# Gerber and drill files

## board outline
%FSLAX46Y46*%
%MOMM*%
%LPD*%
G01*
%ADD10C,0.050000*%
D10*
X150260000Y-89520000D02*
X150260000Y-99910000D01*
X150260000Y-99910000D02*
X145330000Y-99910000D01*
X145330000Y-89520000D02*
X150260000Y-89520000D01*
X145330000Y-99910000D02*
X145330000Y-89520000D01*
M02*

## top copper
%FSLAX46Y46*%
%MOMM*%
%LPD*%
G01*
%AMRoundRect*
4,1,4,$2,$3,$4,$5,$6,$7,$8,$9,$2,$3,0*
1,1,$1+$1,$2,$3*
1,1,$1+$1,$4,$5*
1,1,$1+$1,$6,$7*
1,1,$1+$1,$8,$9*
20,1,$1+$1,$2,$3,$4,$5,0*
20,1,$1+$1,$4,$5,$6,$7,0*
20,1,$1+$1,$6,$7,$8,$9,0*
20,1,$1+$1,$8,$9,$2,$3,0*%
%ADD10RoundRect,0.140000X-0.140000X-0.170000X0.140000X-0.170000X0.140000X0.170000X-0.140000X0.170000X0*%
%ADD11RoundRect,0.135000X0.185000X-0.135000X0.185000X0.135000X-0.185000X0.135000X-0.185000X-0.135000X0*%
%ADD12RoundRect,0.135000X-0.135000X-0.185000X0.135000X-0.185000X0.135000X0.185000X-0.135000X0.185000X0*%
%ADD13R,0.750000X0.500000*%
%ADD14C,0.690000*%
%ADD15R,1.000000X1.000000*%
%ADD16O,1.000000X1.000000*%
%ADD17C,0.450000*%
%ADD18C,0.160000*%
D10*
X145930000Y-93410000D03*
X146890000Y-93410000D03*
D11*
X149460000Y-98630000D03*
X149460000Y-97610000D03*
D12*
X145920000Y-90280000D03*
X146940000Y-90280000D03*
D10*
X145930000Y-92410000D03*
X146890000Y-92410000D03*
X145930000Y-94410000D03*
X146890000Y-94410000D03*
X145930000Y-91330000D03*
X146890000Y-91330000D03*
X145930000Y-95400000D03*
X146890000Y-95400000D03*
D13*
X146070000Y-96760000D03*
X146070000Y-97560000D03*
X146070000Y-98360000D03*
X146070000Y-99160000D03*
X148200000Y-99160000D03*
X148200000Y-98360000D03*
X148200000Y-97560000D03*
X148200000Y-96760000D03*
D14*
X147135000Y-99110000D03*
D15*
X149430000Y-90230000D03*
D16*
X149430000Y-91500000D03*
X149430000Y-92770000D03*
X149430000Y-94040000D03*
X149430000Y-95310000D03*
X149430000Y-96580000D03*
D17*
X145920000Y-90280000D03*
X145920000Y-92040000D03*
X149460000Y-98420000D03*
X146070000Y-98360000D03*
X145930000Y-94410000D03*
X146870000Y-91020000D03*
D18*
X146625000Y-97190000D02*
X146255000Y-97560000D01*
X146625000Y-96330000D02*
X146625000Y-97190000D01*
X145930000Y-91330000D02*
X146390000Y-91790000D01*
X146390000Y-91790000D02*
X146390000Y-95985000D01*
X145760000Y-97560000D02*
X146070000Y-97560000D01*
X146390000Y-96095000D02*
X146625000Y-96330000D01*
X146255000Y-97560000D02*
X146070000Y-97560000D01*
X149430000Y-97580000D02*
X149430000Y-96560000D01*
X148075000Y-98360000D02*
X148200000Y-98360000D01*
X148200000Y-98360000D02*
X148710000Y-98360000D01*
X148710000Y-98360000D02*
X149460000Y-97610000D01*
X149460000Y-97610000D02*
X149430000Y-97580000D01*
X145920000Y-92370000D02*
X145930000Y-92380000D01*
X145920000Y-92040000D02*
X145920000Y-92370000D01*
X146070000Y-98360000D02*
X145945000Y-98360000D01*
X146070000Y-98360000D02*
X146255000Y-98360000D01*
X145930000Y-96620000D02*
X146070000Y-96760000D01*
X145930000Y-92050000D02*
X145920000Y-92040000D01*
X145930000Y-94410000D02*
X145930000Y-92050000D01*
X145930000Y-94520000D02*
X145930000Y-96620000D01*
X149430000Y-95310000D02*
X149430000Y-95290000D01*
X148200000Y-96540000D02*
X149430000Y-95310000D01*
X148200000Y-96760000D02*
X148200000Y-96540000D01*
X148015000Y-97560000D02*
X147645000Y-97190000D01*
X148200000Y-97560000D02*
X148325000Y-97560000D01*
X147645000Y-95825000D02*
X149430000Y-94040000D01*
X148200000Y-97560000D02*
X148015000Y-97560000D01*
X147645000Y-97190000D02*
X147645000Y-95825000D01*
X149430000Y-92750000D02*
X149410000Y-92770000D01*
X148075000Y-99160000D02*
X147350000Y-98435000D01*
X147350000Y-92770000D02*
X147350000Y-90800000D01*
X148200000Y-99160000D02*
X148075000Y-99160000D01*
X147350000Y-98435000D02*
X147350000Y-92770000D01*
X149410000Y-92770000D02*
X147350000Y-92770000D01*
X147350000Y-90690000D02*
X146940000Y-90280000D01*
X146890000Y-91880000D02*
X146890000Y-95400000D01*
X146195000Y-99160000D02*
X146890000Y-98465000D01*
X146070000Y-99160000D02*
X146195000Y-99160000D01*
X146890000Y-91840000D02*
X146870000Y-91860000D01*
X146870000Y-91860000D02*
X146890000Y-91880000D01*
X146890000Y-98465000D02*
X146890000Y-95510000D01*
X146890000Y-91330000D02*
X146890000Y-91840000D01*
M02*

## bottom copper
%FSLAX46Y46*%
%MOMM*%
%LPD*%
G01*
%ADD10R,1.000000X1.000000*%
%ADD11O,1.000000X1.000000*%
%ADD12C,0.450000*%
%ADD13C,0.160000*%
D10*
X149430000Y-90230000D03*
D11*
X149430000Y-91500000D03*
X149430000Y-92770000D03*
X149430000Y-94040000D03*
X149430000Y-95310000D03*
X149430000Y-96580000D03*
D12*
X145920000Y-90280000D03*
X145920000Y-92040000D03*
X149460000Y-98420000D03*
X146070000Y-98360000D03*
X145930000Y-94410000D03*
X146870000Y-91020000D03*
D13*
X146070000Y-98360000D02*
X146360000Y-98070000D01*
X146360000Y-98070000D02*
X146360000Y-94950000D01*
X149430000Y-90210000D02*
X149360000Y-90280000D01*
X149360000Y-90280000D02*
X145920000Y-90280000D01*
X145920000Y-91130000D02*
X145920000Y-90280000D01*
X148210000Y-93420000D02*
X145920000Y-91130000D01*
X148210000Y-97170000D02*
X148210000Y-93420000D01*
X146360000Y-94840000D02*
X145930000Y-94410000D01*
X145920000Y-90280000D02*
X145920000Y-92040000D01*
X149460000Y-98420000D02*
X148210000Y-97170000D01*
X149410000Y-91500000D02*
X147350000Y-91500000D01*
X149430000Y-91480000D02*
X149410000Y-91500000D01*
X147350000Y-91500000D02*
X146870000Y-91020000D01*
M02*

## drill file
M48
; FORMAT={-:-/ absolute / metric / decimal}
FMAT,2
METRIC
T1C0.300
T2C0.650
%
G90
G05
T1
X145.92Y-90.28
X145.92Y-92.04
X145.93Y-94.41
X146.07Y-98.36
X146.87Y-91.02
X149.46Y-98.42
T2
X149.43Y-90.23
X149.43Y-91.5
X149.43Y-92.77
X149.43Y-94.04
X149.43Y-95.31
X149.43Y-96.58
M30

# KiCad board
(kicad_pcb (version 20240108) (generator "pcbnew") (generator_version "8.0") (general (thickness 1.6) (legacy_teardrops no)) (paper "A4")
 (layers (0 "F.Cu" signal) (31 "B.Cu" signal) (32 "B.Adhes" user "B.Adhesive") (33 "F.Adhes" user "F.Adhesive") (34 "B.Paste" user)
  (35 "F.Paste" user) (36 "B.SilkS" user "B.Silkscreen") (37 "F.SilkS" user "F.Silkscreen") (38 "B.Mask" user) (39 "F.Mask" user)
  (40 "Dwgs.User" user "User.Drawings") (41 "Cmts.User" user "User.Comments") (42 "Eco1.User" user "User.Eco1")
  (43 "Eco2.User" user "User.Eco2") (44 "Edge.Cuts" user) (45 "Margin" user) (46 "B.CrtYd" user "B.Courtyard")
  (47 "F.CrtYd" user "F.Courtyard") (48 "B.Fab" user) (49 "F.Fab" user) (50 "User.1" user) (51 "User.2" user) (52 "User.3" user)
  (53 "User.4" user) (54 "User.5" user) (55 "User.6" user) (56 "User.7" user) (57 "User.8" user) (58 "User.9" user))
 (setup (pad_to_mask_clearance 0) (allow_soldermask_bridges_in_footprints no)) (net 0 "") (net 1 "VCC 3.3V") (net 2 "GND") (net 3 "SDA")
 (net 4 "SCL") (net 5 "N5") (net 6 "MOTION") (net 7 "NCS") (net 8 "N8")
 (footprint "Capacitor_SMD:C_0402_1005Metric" (layer "F.Cu") (at 146.41 93.41)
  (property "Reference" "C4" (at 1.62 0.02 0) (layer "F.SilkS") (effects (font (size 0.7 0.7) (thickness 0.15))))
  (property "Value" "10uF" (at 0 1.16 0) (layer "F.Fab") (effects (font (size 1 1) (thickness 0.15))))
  (pad "1" smd roundrect (at -0.48 0) (size 0.56 0.62) (layers "F.Cu" "F.Paste" "F.Mask") (roundrect_rratio 0.25) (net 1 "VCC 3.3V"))
  (pad "2" smd roundrect (at 0.48 0) (size 0.56 0.62) (layers "F.Cu" "F.Paste" "F.Mask") (roundrect_rratio 0.25) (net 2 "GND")))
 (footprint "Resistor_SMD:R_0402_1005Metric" (layer "F.Cu") (at 149.46 98.12 90)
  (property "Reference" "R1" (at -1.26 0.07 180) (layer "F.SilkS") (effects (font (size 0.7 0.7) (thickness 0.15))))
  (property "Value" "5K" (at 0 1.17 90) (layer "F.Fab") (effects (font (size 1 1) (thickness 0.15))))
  (pad "1" smd roundrect (at -0.51 0 90) (size 0.54 0.64) (layers "F.Cu" "F.Paste" "F.Mask") (roundrect_rratio 0.25) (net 1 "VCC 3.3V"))
  (pad "2" smd roundrect (at 0.51 0 90) (size 0.54 0.64) (layers "F.Cu" "F.Paste" "F.Mask") (roundrect_rratio 0.25) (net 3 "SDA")))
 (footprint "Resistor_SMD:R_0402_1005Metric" (layer "F.Cu") (at 146.43 90.28)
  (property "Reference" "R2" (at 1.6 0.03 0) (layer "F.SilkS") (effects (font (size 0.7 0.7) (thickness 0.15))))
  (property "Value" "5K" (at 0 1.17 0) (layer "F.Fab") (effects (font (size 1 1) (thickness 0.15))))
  (pad "1" smd roundrect (at -0.51 0) (size 0.54 0.64) (layers "F.Cu" "F.Paste" "F.Mask") (roundrect_rratio 0.25) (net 1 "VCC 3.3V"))
  (pad "2" smd roundrect (at 0.51 0) (size 0.54 0.64) (layers "F.Cu" "F.Paste" "F.Mask") (roundrect_rratio 0.25) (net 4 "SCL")))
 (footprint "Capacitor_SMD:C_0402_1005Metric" (layer "F.Cu") (at 146.41 92.41)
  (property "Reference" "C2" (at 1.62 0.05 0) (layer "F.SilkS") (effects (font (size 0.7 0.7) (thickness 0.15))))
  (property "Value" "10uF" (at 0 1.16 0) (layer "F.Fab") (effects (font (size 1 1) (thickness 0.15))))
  (pad "1" smd roundrect (at -0.48 0) (size 0.56 0.62) (layers "F.Cu" "F.Paste" "F.Mask") (roundrect_rratio 0.25) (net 1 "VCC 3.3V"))
  (pad "2" smd roundrect (at 0.48 0) (size 0.56 0.62) (layers "F.Cu" "F.Paste" "F.Mask") (roundrect_rratio 0.25) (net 2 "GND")))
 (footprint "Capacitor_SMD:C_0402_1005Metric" (layer "F.Cu") (at 146.41 94.41)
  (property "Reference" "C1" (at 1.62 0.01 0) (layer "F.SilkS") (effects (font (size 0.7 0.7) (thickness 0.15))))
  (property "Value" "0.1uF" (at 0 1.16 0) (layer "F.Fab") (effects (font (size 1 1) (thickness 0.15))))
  (pad "1" smd roundrect (at -0.48 0) (size 0.56 0.62) (layers "F.Cu" "F.Paste" "F.Mask") (roundrect_rratio 0.25) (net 1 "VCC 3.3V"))
  (pad "2" smd roundrect (at 0.48 0) (size 0.56 0.62) (layers "F.Cu" "F.Paste" "F.Mask") (roundrect_rratio 0.25) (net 2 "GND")))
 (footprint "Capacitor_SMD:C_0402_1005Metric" (layer "F.Cu") (at 146.41 91.33)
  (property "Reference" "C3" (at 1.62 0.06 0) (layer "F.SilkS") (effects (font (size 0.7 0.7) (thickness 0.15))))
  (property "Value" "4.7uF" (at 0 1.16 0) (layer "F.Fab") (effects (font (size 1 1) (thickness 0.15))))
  (pad "1" smd roundrect (at -0.48 0) (size 0.56 0.62) (layers "F.Cu" "F.Paste" "F.Mask") (roundrect_rratio 0.25) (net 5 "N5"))
  (pad "2" smd roundrect (at 0.48 0) (size 0.56 0.62) (layers "F.Cu" "F.Paste" "F.Mask") (roundrect_rratio 0.25) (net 2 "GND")))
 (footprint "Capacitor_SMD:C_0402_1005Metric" (layer "F.Cu") (at 146.41 95.4)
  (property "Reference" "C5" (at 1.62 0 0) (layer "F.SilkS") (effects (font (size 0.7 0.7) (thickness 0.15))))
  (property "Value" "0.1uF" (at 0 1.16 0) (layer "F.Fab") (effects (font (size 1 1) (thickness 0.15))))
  (pad "1" smd roundrect (at -0.48 0) (size 0.56 0.62) (layers "F.Cu" "F.Paste" "F.Mask") (roundrect_rratio 0.25) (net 1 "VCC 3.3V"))
  (pad "2" smd roundrect (at 0.48 0) (size 0.56 0.62) (layers "F.Cu" "F.Paste" "F.Mask") (roundrect_rratio 0.25) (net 2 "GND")))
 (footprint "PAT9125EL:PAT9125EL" (layer "F.Cu") (at 147.135 97.96 -90)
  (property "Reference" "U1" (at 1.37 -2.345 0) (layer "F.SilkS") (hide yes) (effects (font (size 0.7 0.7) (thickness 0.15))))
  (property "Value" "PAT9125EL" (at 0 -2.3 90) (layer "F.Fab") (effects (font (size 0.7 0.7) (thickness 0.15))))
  (pad "1" smd rect (at -1.2 1.065 270) (size 0.5 0.75) (layers "F.Cu" "F.Paste" "F.Mask") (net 1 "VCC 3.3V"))
  (pad "2" smd rect (at -0.4 1.065 270) (size 0.5 0.75) (layers "F.Cu" "F.Paste" "F.Mask") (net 5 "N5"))
  (pad "3" smd rect (at 0.4 1.065 270) (size 0.5 0.75) (layers "F.Cu" "F.Paste" "F.Mask") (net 1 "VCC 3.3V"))
  (pad "4" smd rect (at 1.2 1.065 270) (size 0.5 0.75) (layers "F.Cu" "F.Paste" "F.Mask") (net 2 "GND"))
  (pad "5" smd rect (at 1.2 -1.065 270) (size 0.5 0.75) (layers "F.Cu" "F.Paste" "F.Mask") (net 4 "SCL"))
  (pad "6" smd rect (at 0.4 -1.065 270) (size 0.5 0.75) (layers "F.Cu" "F.Paste" "F.Mask") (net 3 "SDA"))
  (pad "7" smd rect (at -0.4 -1.065 270) (size 0.5 0.75) (layers "F.Cu" "F.Paste" "F.Mask") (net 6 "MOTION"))
  (pad "8" smd rect (at -1.2 -1.065 270) (size 0.5 0.75) (layers "F.Cu" "F.Paste" "F.Mask") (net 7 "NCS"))
  (pad "9" smd circle (at 1.15 0 270) (size 0.69 0.69) (layers "F.Cu" "F.Paste" "F.Mask") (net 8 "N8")))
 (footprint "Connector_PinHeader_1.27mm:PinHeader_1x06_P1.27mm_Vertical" (layer "F.Cu") (at 149.43 90.23)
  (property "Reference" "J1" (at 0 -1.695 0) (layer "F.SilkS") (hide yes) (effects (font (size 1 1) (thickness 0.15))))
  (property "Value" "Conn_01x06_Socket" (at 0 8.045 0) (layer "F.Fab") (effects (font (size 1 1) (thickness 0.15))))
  (pad "1" thru_hole rect (at 0 0) (size 1 1) (drill 0.65) (layers "*.Cu" "*.Mask") (remove_unused_layers no) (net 1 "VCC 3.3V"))
  (pad "2" thru_hole oval (at 0 1.27) (size 1 1) (drill 0.65) (layers "*.Cu" "*.Mask") (remove_unused_layers no) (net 2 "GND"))
  (pad "3" thru_hole oval (at 0 2.54) (size 1 1) (drill 0.65) (layers "*.Cu" "*.Mask") (remove_unused_layers no) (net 4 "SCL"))
  (pad "4" thru_hole oval (at 0 3.81) (size 1 1) (drill 0.65) (layers "*.Cu" "*.Mask") (remove_unused_layers no) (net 6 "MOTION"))
  (pad "5" thru_hole oval (at 0 5.08) (size 1 1) (drill 0.65) (layers "*.Cu" "*.Mask") (remove_unused_layers no) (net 7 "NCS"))
  (pad "6" thru_hole oval (at 0 6.35) (size 1 1) (drill 0.65) (layers "*.Cu" "*.Mask") (remove_unused_layers no) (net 3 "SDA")))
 (gr_line (start 150.26 89.52) (end 150.26 99.91) (stroke (width 0.05) (type default)) (layer "Edge.Cuts"))
 (gr_line (start 150.26 99.91) (end 145.33 99.91) (stroke (width 0.05) (type default)) (layer "Edge.Cuts"))
 (gr_line (start 145.33 89.52) (end 150.26 89.52) (stroke (width 0.05) (type default)) (layer "Edge.Cuts"))
 (gr_line (start 145.33 99.91) (end 145.33 89.52) (stroke (width 0.05) (type default)) (layer "Edge.Cuts"))
 (segment (start 146.625 97.19) (end 146.255 97.56) (width 0.16) (layer "F.Cu") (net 5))
 (segment (start 146.625 96.33) (end 146.625 97.19) (width 0.16) (layer "F.Cu") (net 5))
 (segment (start 145.93 91.33) (end 146.39 91.79) (width 0.16) (layer "F.Cu") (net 5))
 (segment (start 146.39 91.79) (end 146.39 95.985) (width 0.16) (layer "F.Cu") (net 5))
 (segment (start 145.76 97.56) (end 146.07 97.56) (width 0.16) (layer "F.Cu") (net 5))
 (segment (start 146.39 96.095) (end 146.625 96.33) (width 0.16) (layer "F.Cu") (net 5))
 (segment (start 146.255 97.56) (end 146.07 97.56) (width 0.16) (layer "F.Cu") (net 5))
 (segment (start 149.43 97.58) (end 149.43 96.56) (width 0.16) (layer "F.Cu") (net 3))
 (segment (start 148.075 98.36) (end 148.2 98.36) (width 0.16) (layer "F.Cu") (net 3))
 (segment (start 148.2 98.36) (end 148.71 98.36) (width 0.16) (layer "F.Cu") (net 3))
 (segment (start 148.71 98.36) (end 149.46 97.61) (width 0.16) (layer "F.Cu") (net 3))
 (segment (start 149.46 97.61) (end 149.43 97.58) (width 0.16) (layer "F.Cu") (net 3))
 (segment (start 145.92 92.37) (end 145.93 92.38) (width 0.16) (layer "F.Cu") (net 1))
 (segment (start 145.92 92.04) (end 145.92 92.37) (width 0.16) (layer "F.Cu") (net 1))
 (segment (start 146.07 98.36) (end 145.945 98.36) (width 0.16) (layer "F.Cu") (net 1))
 (segment (start 146.07 98.36) (end 146.255 98.36) (width 0.16) (layer "F.Cu") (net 1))
 (segment (start 145.93 96.62) (end 146.07 96.76) (width 0.16) (layer "F.Cu") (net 1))
 (segment (start 145.93 92.05) (end 145.92 92.04) (width 0.16) (layer "F.Cu") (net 1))
 (segment (start 145.93 94.41) (end 145.93 92.05) (width 0.16) (layer "F.Cu") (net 1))
 (segment (start 145.93 94.52) (end 145.93 96.62) (width 0.16) (layer "F.Cu") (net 1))
 (via (at 145.92 90.28) (size 0.45) (drill 0.3) (layers "F.Cu" "B.Cu") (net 1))
 (via (at 145.92 92.04) (size 0.45) (drill 0.3) (layers "F.Cu" "B.Cu") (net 1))
 (via (at 149.46 98.42) (size 0.45) (drill 0.3) (layers "F.Cu" "B.Cu") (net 1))
 (via (at 146.07 98.36) (size 0.45) (drill 0.3) (layers "F.Cu" "B.Cu") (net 1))
 (via (at 145.93 94.41) (size 0.45) (drill 0.3) (layers "F.Cu" "B.Cu") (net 1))
 (segment (start 146.07 98.36) (end 146.36 98.07) (width 0.16) (layer "B.Cu") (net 1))
 (segment (start 146.36 98.07) (end 146.36 94.95) (width 0.16) (layer "B.Cu") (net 1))
 (segment (start 149.43 90.21) (end 149.36 90.28) (width 0.16) (layer "B.Cu") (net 1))
 (segment (start 149.36 90.28) (end 145.92 90.28) (width 0.16) (layer "B.Cu") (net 1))
 (segment (start 145.92 91.13) (end 145.92 90.28) (width 0.16) (layer "B.Cu") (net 1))
 (segment (start 148.21 93.42) (end 145.92 91.13) (width 0.16) (layer "B.Cu") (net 1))
 (segment (start 148.21 97.17) (end 148.21 93.42) (width 0.16) (layer "B.Cu") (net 1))
 (segment (start 146.36 94.84) (end 145.93 94.41) (width 0.16) (layer "B.Cu") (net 1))
 (segment (start 145.92 90.28) (end 145.92 92.04) (width 0.16) (layer "B.Cu") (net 1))
 (segment (start 149.46 98.42) (end 148.21 97.17) (width 0.16) (layer "B.Cu") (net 1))
 (segment (start 149.43 95.31) (end 149.43 95.29) (width 0.16) (layer "F.Cu") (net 7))
 (segment (start 148.2 96.54) (end 149.43 95.31) (width 0.16) (layer "F.Cu") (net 7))
 (segment (start 148.2 96.76) (end 148.2 96.54) (width 0.16) (layer "F.Cu") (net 7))
 (segment (start 148.015 97.56) (end 147.645 97.19) (width 0.16) (layer "F.Cu") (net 6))
 (segment (start 148.2 97.56) (end 148.325 97.56) (width 0.16) (layer "F.Cu") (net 6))
 (segment (start 147.645 95.825) (end 149.43 94.04) (width 0.16) (layer "F.Cu") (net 6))
 (segment (start 148.2 97.56) (end 148.015 97.56) (width 0.16) (layer "F.Cu") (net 6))
 (segment (start 147.645 97.19) (end 147.645 95.825) (width 0.16) (layer "F.Cu") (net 6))
 (segment (start 149.43 92.75) (end 149.41 92.77) (width 0.16) (layer "F.Cu") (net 4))
 (segment (start 148.075 99.16) (end 147.35 98.435) (width 0.16) (layer "F.Cu") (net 4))
 (segment (start 147.35 92.77) (end 147.35 90.8) (width 0.16) (layer "F.Cu") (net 4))
 (segment (start 148.2 99.16) (end 148.075 99.16) (width 0.16) (layer "F.Cu") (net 4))
 (segment (start 147.35 98.435) (end 147.35 92.77) (width 0.16) (layer "F.Cu") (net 4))
 (segment (start 149.41 92.77) (end 147.35 92.77) (width 0.16) (layer "F.Cu") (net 4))
 (segment (start 147.35 90.69) (end 146.94 90.28) (width 0.16) (layer "F.Cu") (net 4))
 (segment (start 146.89 91.88) (end 146.89 95.4) (width 0.16) (layer "F.Cu") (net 2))
 (segment (start 146.195 99.16) (end 146.89 98.465) (width 0.16) (layer "F.Cu") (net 2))
 (segment (start 146.07 99.16) (end 146.195 99.16) (width 0.16) (layer "F.Cu") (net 2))
 (segment (start 146.89 91.84) (end 146.87 91.86) (width 0.16) (layer "F.Cu") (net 2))
 (segment (start 146.87 91.86) (end 146.89 91.88) (width 0.16) (layer "F.Cu") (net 2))
 (segment (start 146.89 98.465) (end 146.89 95.51) (width 0.16) (layer "F.Cu") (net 2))
 (segment (start 146.89 91.33) (end 146.89 91.84) (width 0.16) (layer "F.Cu") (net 2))
 (via (at 146.87 91.02) (size 0.45) (drill 0.3) (layers "F.Cu" "B.Cu") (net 2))
 (segment (start 149.41 91.5) (end 147.35 91.5) (width 0.16) (layer "B.Cu") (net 2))
 (segment (start 149.43 91.48) (end 149.41 91.5) (width 0.16) (layer "B.Cu") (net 2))
 (segment (start 147.35 91.5) (end 146.87 91.02) (width 0.16) (layer "B.Cu") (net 2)))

